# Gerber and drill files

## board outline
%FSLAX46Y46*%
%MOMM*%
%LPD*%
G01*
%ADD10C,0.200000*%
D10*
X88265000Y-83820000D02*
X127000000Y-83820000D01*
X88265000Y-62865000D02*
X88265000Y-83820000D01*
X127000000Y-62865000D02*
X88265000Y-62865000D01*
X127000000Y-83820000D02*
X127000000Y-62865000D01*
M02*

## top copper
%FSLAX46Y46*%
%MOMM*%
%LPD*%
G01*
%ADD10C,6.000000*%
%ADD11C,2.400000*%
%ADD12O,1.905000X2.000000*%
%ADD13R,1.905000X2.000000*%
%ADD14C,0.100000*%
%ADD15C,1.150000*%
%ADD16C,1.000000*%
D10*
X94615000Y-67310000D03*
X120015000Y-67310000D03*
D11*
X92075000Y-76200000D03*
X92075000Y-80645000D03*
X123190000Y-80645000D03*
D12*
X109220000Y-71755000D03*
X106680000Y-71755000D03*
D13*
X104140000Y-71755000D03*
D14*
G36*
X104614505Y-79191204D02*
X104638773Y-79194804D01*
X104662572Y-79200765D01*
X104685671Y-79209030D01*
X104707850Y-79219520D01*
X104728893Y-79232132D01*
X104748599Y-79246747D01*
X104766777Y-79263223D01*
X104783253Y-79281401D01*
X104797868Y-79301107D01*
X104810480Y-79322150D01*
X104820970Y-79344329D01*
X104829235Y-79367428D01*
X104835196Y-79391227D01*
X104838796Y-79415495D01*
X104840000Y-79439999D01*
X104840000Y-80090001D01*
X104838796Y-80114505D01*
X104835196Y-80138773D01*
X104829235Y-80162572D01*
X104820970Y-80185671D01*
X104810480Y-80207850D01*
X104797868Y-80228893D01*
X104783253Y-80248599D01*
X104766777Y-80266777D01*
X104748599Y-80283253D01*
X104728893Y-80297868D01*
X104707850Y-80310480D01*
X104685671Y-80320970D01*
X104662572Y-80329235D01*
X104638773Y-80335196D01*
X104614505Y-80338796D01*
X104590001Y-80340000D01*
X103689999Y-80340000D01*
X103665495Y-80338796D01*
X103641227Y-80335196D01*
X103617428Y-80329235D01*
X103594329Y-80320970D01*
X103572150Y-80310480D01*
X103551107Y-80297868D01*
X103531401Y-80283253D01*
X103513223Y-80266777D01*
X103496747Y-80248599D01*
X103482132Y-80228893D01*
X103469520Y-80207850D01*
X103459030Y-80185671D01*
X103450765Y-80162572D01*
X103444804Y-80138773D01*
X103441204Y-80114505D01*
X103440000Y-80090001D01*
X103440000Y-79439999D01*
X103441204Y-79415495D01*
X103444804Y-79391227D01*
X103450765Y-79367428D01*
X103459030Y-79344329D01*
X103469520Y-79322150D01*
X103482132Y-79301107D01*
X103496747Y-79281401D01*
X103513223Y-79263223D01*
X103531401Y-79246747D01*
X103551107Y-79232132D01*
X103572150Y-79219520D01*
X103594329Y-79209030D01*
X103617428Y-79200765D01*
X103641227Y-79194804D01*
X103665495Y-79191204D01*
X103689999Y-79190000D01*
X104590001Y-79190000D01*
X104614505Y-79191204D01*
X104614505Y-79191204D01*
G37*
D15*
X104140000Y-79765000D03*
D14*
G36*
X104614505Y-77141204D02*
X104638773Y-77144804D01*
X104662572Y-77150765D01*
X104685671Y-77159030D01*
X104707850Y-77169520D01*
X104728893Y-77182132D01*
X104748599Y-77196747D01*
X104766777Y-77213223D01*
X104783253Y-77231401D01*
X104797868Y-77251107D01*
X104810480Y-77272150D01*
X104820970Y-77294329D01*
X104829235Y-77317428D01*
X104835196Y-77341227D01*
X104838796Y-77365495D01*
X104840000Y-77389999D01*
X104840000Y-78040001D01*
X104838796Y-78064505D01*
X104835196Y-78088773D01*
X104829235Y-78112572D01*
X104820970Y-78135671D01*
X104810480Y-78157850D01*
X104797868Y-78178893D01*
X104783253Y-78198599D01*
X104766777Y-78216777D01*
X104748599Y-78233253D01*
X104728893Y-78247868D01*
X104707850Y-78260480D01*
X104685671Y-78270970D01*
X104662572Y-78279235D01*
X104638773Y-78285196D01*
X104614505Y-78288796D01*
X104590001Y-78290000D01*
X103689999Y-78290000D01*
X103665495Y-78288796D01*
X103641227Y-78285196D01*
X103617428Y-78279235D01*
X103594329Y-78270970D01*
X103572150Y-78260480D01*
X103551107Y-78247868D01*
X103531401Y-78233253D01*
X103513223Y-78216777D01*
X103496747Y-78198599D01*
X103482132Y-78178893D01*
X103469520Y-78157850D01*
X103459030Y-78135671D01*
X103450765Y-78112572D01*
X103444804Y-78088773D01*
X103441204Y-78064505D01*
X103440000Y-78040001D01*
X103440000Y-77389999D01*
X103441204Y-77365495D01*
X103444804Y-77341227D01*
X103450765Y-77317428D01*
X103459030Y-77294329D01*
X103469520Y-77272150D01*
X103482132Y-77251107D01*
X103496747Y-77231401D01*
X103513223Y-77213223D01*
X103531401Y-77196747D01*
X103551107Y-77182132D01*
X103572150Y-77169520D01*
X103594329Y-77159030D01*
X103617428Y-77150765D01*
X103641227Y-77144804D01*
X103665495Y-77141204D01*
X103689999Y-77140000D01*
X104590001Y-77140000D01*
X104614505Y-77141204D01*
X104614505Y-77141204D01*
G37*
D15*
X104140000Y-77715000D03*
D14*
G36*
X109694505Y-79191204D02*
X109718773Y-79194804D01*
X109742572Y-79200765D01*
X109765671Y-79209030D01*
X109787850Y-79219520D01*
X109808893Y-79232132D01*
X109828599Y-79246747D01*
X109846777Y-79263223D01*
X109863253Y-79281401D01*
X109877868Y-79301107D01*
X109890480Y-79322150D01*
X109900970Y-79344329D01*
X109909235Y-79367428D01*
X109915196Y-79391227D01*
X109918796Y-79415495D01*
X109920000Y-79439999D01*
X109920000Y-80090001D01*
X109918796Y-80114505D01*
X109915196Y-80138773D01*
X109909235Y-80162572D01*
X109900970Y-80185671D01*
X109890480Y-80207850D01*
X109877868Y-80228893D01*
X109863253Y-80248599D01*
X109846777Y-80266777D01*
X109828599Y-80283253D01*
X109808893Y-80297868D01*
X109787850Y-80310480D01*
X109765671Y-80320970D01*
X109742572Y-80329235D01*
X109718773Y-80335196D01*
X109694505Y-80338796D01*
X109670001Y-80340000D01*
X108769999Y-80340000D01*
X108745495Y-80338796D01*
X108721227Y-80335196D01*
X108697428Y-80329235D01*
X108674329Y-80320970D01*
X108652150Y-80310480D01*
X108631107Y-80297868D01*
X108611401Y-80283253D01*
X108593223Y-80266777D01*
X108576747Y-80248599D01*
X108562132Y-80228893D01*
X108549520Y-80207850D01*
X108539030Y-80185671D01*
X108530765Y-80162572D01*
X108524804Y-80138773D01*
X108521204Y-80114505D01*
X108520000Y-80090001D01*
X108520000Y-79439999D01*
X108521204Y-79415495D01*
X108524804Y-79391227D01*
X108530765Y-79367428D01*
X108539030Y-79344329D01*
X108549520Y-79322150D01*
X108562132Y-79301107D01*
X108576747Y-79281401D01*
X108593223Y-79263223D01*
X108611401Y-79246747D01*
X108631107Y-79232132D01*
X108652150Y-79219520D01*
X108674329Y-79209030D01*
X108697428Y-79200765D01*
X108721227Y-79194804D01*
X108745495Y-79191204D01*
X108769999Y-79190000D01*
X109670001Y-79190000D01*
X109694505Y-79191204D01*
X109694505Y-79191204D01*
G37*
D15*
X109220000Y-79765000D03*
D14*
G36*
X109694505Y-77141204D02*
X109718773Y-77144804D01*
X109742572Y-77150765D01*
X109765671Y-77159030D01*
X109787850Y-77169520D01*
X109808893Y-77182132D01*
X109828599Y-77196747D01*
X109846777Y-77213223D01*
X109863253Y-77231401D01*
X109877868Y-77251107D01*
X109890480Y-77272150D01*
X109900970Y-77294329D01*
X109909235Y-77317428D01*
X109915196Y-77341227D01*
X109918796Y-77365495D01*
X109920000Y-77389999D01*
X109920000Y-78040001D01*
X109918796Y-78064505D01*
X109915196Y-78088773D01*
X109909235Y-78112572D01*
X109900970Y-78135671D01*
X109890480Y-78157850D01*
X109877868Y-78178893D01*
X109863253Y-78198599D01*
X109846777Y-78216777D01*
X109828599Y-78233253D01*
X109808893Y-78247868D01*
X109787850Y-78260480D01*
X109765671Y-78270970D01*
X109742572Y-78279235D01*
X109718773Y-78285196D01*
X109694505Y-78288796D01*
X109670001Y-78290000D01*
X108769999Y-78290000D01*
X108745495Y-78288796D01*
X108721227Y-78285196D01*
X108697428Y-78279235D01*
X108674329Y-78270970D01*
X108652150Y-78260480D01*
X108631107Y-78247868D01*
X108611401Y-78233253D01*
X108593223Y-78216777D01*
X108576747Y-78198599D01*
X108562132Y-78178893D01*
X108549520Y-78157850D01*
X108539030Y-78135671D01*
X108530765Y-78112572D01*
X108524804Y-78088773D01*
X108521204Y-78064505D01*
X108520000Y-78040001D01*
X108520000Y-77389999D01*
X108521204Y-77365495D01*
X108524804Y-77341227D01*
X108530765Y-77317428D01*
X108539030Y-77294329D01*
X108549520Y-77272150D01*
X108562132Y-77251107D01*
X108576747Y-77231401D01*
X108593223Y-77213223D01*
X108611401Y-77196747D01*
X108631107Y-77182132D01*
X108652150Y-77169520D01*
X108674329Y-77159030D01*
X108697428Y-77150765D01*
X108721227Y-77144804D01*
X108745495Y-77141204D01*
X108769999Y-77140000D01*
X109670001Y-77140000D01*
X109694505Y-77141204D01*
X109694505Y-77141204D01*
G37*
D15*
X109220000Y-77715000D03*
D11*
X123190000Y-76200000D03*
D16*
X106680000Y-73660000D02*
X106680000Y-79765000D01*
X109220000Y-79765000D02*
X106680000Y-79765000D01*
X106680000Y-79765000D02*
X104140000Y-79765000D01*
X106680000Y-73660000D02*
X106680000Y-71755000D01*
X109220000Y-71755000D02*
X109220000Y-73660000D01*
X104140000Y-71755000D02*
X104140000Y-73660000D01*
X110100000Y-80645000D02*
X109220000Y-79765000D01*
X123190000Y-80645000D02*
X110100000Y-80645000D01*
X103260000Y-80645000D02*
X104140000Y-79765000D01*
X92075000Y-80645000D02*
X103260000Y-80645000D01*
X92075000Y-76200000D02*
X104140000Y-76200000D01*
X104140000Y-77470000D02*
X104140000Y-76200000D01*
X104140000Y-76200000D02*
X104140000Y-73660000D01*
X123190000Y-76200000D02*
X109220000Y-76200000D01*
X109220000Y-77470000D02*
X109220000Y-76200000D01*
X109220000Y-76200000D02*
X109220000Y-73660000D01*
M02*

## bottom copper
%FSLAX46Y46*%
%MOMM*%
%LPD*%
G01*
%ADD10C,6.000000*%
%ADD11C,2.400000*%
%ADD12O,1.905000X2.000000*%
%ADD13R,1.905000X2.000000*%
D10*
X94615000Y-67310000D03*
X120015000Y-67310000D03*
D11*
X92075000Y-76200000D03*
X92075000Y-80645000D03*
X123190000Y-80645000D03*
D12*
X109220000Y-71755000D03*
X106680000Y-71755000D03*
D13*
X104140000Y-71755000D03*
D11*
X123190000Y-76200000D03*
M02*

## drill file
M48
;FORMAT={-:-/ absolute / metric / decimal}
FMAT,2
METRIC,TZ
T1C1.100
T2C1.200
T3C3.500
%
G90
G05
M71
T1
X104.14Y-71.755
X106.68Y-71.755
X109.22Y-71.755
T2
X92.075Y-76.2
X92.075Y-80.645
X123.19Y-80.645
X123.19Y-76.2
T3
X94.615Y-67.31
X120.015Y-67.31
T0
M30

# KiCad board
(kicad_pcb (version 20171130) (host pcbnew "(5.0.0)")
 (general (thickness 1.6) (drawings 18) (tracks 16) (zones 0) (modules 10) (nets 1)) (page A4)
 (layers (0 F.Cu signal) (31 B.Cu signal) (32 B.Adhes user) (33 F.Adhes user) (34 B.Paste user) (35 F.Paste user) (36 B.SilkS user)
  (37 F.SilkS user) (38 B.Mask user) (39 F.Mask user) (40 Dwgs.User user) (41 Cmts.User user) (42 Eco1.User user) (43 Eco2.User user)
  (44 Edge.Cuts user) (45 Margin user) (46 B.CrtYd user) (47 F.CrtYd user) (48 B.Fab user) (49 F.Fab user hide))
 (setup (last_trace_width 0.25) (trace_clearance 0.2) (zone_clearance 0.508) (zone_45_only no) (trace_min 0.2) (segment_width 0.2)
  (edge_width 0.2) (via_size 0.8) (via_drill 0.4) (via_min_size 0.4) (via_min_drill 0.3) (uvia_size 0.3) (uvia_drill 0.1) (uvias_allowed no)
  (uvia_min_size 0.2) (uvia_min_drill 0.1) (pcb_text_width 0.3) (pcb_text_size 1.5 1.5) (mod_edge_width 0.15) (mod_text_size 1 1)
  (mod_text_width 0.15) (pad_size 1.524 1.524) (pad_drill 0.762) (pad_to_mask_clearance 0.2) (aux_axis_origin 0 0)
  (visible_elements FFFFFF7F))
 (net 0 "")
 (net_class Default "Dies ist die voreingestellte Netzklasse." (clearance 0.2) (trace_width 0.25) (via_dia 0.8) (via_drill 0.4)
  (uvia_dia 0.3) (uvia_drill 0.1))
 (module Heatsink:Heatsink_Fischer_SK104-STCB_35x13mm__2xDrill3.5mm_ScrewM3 (layer F.Cu) (at 107.315 67.31)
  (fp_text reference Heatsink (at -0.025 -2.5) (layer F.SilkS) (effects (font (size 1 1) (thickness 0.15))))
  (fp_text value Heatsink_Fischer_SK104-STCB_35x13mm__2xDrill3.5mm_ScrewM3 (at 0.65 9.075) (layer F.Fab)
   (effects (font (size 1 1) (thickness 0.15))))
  (pad 1 thru_hole circle (at -12.7 0 180) (size 6 6) (drill 3.5) (layers *.Cu *.Mask))
  (pad 1 thru_hole circle (at 12.7 0) (size 6 6) (drill 3.5) (layers *.Cu *.Mask)))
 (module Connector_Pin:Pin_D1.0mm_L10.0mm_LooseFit (layer F.Cu) (at 92.075 76.2)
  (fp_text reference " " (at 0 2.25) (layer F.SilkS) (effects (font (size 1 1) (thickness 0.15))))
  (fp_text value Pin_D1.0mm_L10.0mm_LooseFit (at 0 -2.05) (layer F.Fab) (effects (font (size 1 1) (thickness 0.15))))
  (pad 1 thru_hole circle (at 0 0) (size 2.4 2.4) (drill 1.2) (layers *.Cu *.Mask)))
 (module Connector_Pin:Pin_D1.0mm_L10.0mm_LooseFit (layer F.Cu) (at 92.075 80.645)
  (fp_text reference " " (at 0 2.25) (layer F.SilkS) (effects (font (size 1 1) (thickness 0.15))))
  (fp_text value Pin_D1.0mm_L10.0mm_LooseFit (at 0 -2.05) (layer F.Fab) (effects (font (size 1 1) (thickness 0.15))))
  (pad 1 thru_hole circle (at 0 0) (size 2.4 2.4) (drill 1.2) (layers *.Cu *.Mask)))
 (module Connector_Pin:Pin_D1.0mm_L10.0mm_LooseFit (layer F.Cu) (at 123.19 80.645)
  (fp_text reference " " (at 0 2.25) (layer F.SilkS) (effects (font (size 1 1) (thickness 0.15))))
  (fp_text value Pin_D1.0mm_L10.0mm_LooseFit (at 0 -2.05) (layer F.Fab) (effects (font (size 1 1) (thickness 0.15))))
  (pad 1 thru_hole circle (at 0 0) (size 2.4 2.4) (drill 1.2) (layers *.Cu *.Mask)))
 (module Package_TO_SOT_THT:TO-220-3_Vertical (layer F.Cu) (at 104.14 71.755)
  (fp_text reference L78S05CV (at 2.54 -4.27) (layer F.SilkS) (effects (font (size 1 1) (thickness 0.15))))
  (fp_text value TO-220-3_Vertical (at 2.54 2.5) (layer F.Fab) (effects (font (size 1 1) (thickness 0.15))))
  (pad 3 thru_hole oval (at 5.08 0) (size 1.905 2) (drill 1.1) (layers *.Cu *.Mask))
  (pad 2 thru_hole oval (at 2.54 0) (size 1.905 2) (drill 1.1) (layers *.Cu *.Mask))
  (pad 1 thru_hole rect (at 0 0) (size 1.905 2) (drill 1.1) (layers *.Cu *.Mask)))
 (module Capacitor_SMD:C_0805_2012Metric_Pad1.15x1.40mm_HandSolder (layer F.Cu) (at 104.14 78.74 270)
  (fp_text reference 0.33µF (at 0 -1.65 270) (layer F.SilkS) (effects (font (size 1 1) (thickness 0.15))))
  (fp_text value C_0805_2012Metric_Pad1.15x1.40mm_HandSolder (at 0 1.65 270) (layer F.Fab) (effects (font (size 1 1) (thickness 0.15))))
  (pad 2 smd roundrect (at 1.025 0 270) (size 1.15 1.4) (layers F.Cu F.Paste F.Mask) (roundrect_rratio 0.217391))
  (pad 1 smd roundrect (at -1.025 0 270) (size 1.15 1.4) (layers F.Cu F.Paste F.Mask) (roundrect_rratio 0.217391)))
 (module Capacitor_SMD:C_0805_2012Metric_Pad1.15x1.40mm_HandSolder (layer F.Cu) (at 109.22 78.74 270)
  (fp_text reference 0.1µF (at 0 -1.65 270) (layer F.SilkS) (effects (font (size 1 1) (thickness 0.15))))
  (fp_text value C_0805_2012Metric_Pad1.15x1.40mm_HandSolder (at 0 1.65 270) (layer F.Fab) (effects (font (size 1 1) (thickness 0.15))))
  (pad 2 smd roundrect (at 1.025 0 270) (size 1.15 1.4) (layers F.Cu F.Paste F.Mask) (roundrect_rratio 0.217391))
  (pad 1 smd roundrect (at -1.025 0 270) (size 1.15 1.4) (layers F.Cu F.Paste F.Mask) (roundrect_rratio 0.217391)))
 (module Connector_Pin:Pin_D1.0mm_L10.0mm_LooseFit (layer F.Cu) (at 123.19 76.2)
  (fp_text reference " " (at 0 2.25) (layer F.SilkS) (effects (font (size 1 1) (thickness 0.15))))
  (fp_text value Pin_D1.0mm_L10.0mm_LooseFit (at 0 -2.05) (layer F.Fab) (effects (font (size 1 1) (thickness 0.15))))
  (pad 1 thru_hole circle (at 0 0) (size 2.4 2.4) (drill 1.2) (layers *.Cu *.Mask)))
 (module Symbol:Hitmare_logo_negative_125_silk (layer F.Cu) (at 115.57 73.66)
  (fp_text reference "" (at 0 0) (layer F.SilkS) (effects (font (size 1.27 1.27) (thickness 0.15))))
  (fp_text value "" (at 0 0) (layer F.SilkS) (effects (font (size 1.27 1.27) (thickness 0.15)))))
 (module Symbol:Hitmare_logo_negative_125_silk (layer B.Cu) (at 99.06 73.66 180)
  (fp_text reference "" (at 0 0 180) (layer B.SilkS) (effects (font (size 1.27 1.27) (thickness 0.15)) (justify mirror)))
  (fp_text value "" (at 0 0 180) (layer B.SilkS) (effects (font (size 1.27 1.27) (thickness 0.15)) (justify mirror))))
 (gr_line (start 88.265 83.82) (end 127 83.82) (layer Edge.Cuts) (width 0.2))
 (gr_line (start 88.265 62.865) (end 88.265 83.82) (layer Edge.Cuts) (width 0.2))
 (gr_line (start 127 62.865) (end 88.265 62.865) (layer Edge.Cuts) (width 0.2))
 (gr_line (start 127 83.82) (end 127 62.865) (layer Edge.Cuts) (width 0.2))
 (segment (start 106.68 73.66) (end 106.68 79.765) (width 1) (layer F.Cu) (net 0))
 (segment (start 109.22 79.765) (end 106.68 79.765) (width 1) (layer F.Cu) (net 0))
 (segment (start 106.68 79.765) (end 104.14 79.765) (width 1) (layer F.Cu) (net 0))
 (segment (start 106.68 73.66) (end 106.68 71.755) (width 1) (layer F.Cu) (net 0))
 (segment (start 109.22 71.755) (end 109.22 73.66) (width 1) (layer F.Cu) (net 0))
 (segment (start 104.14 71.755) (end 104.14 73.66) (width 1) (layer F.Cu) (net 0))
 (segment (start 110.1 80.645) (end 109.22 79.765) (width 1) (layer F.Cu) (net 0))
 (segment (start 123.19 80.645) (end 110.1 80.645) (width 1) (layer F.Cu) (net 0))
 (segment (start 103.26 80.645) (end 104.14 79.765) (width 1) (layer F.Cu) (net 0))
 (segment (start 92.075 80.645) (end 103.26 80.645) (width 1) (layer F.Cu) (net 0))
 (segment (start 92.075 76.2) (end 104.14 76.2) (width 1) (layer F.Cu) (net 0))
 (segment (start 104.14 77.47) (end 104.14 76.2) (width 1) (layer F.Cu) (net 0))
 (segment (start 104.14 76.2) (end 104.14 73.66) (width 1) (layer F.Cu) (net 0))
 (segment (start 123.19 76.2) (end 109.22 76.2) (width 1) (layer F.Cu) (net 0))
 (segment (start 109.22 77.47) (end 109.22 76.2) (width 1) (layer F.Cu) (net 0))
 (segment (start 109.22 76.2) (end 109.22 73.66) (width 1) (layer F.Cu) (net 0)))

